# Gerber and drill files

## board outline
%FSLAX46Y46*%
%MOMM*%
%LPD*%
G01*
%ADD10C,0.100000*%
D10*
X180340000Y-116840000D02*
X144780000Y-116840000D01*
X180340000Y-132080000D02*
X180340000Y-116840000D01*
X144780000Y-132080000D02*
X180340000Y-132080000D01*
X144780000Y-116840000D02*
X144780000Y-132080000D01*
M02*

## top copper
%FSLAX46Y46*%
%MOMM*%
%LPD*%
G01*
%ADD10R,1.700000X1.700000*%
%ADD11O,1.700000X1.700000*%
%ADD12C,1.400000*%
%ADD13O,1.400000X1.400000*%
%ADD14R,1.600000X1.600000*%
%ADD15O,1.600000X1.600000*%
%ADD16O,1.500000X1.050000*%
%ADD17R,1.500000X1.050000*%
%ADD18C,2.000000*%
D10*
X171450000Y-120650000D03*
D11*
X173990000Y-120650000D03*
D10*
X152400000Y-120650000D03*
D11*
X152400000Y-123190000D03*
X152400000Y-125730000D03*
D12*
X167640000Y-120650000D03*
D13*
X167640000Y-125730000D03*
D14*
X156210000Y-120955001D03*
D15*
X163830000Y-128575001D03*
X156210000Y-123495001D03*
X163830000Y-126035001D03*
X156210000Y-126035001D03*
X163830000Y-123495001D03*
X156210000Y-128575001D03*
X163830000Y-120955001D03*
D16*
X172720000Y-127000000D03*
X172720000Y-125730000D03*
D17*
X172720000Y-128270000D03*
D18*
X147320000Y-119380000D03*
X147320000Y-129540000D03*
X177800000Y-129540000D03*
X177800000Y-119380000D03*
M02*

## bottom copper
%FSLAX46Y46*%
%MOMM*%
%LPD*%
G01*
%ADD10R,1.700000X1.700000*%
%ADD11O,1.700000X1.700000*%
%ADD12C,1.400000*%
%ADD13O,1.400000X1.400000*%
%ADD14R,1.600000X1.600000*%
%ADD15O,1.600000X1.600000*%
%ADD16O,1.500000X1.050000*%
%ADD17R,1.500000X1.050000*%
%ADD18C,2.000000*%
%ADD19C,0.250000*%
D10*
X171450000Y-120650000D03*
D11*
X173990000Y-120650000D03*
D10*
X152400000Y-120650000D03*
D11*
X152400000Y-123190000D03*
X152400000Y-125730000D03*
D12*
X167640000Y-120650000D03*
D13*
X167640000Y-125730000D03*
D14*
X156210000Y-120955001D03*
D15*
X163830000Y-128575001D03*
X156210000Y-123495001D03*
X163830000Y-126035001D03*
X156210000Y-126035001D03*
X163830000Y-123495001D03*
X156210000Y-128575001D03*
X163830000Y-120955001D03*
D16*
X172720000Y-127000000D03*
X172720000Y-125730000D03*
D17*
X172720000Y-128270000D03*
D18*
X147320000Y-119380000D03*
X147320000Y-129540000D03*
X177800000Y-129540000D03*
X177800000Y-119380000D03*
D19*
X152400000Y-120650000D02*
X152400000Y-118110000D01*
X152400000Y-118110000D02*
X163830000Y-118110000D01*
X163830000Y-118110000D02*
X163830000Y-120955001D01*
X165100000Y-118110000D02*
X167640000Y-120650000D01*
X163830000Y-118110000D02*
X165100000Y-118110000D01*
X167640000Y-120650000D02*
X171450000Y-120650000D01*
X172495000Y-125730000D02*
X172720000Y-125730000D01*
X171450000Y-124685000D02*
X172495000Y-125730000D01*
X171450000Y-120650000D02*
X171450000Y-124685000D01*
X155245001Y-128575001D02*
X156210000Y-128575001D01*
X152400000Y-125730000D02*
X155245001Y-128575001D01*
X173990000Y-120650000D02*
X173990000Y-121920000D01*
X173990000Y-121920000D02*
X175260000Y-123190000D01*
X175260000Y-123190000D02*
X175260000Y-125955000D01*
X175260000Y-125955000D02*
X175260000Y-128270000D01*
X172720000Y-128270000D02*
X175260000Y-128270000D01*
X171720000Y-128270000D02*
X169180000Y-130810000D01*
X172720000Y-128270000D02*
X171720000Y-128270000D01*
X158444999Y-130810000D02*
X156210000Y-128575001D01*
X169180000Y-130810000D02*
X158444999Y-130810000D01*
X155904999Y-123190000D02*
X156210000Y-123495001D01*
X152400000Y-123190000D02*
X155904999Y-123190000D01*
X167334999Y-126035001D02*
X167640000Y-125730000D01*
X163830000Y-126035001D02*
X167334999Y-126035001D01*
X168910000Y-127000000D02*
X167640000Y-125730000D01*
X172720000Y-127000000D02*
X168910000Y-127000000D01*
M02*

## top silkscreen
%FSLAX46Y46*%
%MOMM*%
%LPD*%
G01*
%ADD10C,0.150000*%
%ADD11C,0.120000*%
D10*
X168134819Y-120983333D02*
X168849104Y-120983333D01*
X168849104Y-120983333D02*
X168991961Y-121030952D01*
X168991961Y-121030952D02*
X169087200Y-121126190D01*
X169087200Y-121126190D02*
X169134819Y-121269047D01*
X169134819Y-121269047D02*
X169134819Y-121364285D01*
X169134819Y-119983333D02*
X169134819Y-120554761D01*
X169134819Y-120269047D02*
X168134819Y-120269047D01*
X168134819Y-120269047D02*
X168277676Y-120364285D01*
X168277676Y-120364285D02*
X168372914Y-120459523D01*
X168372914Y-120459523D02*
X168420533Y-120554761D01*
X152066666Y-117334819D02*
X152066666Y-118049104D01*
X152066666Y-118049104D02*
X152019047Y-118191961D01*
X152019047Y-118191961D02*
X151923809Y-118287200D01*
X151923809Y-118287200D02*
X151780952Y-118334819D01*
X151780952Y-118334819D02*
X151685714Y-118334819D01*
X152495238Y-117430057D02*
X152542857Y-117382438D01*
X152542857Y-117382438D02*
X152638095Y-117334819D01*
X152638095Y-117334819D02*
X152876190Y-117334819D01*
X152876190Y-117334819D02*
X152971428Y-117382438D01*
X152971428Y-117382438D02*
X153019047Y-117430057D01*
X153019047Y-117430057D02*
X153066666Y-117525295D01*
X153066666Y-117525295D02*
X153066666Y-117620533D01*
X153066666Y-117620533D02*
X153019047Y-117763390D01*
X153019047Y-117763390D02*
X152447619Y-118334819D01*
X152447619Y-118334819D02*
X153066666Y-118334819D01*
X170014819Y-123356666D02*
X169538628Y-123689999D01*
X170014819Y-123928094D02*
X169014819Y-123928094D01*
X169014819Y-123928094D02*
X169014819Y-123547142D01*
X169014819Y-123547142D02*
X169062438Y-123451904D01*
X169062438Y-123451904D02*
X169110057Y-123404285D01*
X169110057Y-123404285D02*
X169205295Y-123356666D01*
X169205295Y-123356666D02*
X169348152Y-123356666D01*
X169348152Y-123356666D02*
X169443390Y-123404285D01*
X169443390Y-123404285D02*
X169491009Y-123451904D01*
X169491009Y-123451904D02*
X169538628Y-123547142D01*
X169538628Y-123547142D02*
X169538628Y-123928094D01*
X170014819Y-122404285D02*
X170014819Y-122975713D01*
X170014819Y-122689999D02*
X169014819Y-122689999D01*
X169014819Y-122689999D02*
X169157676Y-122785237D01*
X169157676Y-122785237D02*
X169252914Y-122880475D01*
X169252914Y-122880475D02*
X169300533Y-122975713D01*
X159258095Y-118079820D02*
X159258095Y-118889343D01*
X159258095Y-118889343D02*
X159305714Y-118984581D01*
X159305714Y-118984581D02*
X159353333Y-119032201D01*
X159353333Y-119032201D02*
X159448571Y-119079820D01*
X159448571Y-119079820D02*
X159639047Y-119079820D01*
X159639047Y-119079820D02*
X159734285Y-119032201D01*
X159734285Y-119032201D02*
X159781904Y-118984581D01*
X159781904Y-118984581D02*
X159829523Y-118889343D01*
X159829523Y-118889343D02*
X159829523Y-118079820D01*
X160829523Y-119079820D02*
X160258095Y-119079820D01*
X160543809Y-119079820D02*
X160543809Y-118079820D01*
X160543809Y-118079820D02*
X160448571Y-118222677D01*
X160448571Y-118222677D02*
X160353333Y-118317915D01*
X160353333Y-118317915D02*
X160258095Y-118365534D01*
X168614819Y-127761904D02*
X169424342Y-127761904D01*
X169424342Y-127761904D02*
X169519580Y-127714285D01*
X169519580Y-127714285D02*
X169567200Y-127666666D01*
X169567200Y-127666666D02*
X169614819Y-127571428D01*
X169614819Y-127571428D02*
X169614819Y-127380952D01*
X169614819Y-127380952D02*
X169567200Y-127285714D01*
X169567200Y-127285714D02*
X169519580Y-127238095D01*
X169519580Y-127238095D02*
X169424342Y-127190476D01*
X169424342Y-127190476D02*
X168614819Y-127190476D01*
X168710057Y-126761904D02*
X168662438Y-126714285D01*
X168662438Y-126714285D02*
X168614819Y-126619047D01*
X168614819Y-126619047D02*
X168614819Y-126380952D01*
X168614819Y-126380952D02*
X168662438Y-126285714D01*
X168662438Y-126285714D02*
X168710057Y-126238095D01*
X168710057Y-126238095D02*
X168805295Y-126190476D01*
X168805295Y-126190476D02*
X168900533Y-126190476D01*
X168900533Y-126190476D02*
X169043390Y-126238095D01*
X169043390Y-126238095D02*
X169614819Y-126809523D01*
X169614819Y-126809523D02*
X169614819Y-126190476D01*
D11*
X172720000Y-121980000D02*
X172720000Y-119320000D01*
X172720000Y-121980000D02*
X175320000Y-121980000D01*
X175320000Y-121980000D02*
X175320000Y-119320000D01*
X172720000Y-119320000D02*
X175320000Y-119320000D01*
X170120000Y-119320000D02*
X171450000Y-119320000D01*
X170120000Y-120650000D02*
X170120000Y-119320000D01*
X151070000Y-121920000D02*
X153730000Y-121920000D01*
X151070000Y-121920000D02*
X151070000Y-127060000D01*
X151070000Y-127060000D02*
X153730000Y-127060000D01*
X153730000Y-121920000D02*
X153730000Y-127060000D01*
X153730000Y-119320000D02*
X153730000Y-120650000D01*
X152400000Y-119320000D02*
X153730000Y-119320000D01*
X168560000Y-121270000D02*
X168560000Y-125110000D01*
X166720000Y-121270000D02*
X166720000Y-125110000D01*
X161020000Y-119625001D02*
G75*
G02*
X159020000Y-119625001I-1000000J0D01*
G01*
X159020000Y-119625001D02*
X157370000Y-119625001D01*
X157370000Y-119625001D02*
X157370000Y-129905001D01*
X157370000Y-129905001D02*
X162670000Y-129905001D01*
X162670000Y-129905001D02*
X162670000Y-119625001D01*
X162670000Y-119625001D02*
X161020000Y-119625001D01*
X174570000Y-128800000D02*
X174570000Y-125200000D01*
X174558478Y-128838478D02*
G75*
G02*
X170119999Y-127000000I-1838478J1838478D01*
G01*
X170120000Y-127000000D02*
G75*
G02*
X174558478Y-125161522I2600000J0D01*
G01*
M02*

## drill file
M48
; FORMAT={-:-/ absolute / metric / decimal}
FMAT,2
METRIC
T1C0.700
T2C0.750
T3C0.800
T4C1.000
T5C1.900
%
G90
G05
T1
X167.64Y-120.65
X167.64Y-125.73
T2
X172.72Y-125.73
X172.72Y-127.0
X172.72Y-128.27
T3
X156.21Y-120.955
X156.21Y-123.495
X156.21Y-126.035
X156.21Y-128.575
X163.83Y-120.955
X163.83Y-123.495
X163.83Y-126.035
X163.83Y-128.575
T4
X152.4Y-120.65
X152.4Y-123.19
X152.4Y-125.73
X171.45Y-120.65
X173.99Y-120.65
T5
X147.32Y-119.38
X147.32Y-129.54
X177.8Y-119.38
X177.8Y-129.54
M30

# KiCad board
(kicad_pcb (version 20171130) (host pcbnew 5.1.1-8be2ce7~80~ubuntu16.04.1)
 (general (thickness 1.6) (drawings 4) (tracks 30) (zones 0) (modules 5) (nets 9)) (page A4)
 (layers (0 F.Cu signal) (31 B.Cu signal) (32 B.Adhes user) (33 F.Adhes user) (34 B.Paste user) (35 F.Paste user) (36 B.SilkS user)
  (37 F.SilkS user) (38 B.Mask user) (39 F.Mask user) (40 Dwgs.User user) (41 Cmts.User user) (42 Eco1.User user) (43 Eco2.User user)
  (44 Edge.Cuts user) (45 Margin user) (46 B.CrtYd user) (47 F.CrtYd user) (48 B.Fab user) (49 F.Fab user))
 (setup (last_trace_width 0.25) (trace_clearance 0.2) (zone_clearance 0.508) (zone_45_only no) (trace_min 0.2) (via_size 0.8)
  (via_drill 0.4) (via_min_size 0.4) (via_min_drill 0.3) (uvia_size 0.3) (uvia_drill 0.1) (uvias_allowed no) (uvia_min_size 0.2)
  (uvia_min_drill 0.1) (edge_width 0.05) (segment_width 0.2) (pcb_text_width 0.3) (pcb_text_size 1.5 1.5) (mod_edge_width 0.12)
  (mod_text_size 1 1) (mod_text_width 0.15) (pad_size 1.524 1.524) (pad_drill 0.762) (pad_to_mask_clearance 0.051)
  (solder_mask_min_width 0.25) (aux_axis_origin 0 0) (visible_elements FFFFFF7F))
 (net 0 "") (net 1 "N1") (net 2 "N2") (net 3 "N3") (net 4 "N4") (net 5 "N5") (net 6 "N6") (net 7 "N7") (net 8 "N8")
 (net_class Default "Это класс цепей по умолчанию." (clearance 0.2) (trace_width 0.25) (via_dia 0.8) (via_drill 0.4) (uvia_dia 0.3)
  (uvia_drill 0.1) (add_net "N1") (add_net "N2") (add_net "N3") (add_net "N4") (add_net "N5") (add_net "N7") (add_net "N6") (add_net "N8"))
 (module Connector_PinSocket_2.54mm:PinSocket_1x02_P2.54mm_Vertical (layer F.Cu) (at 171.45 120.65 90)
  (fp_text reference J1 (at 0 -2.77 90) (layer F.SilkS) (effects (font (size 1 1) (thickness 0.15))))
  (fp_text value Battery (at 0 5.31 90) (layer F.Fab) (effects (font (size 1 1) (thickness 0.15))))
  (fp_line (start -1.33 1.27) (end 1.33 1.27) (layer F.SilkS) (width 0.12))
  (fp_line (start -1.33 1.27) (end -1.33 3.87) (layer F.SilkS) (width 0.12))
  (fp_line (start -1.33 3.87) (end 1.33 3.87) (layer F.SilkS) (width 0.12))
  (fp_line (start 1.33 1.27) (end 1.33 3.87) (layer F.SilkS) (width 0.12))
  (fp_line (start 1.33 -1.33) (end 1.33 0) (layer F.SilkS) (width 0.12))
  (fp_line (start 0 -1.33) (end 1.33 -1.33) (layer F.SilkS) (width 0.12))
  (pad 1 thru_hole rect (at 0 0 90) (size 1.7 1.7) (drill 1) (layers *.Cu *.Mask) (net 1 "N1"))
  (pad 2 thru_hole oval (at 0 2.54 90) (size 1.7 1.7) (drill 1) (layers *.Cu *.Mask) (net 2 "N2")))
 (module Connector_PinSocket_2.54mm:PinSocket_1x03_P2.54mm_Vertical (layer F.Cu) (at 152.4 120.65)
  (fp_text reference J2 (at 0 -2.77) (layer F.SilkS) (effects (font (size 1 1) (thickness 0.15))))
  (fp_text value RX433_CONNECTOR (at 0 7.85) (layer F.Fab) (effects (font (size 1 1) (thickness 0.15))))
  (fp_line (start -1.33 1.27) (end 1.33 1.27) (layer F.SilkS) (width 0.12))
  (fp_line (start -1.33 1.27) (end -1.33 6.41) (layer F.SilkS) (width 0.12))
  (fp_line (start -1.33 6.41) (end 1.33 6.41) (layer F.SilkS) (width 0.12))
  (fp_line (start 1.33 1.27) (end 1.33 6.41) (layer F.SilkS) (width 0.12))
  (fp_line (start 1.33 -1.33) (end 1.33 0) (layer F.SilkS) (width 0.12))
  (fp_line (start 0 -1.33) (end 1.33 -1.33) (layer F.SilkS) (width 0.12))
  (pad 1 thru_hole rect (at 0 0) (size 1.7 1.7) (drill 1) (layers *.Cu *.Mask) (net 1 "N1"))
  (pad 2 thru_hole oval (at 0 2.54) (size 1.7 1.7) (drill 1) (layers *.Cu *.Mask) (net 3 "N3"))
  (pad 3 thru_hole oval (at 0 5.08) (size 1.7 1.7) (drill 1) (layers *.Cu *.Mask) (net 2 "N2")))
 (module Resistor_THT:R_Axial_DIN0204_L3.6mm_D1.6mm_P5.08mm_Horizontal (layer F.Cu) (at 167.64 120.65 270)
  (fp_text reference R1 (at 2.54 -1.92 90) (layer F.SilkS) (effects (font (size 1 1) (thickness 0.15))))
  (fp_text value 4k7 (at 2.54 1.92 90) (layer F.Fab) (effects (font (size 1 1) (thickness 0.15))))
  (fp_line (start 0.62 -0.92) (end 4.46 -0.92) (layer F.SilkS) (width 0.12))
  (fp_line (start 0.62 0.92) (end 4.46 0.92) (layer F.SilkS) (width 0.12))
  (pad 1 thru_hole circle (at 0 0 270) (size 1.4 1.4) (drill 0.7) (layers *.Cu *.Mask) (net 1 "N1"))
  (pad 2 thru_hole oval (at 5.08 0 270) (size 1.4 1.4) (drill 0.7) (layers *.Cu *.Mask) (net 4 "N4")))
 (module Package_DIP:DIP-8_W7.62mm (layer F.Cu) (at 156.21 120.955001)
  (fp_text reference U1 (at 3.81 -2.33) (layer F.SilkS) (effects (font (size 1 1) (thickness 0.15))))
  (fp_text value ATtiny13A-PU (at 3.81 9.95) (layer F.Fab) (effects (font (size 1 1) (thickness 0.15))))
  (fp_arc (start 3.81 -1.33) (end 2.81 -1.33) (angle -180) (layer F.SilkS) (width 0.12))
  (fp_line (start 2.81 -1.33) (end 1.16 -1.33) (layer F.SilkS) (width 0.12))
  (fp_line (start 1.16 -1.33) (end 1.16 8.95) (layer F.SilkS) (width 0.12))
  (fp_line (start 1.16 8.95) (end 6.46 8.95) (layer F.SilkS) (width 0.12))
  (fp_line (start 6.46 8.95) (end 6.46 -1.33) (layer F.SilkS) (width 0.12))
  (fp_line (start 6.46 -1.33) (end 4.81 -1.33) (layer F.SilkS) (width 0.12))
  (pad 1 thru_hole rect (at 0 0) (size 1.6 1.6) (drill 0.8) (layers *.Cu *.Mask) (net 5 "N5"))
  (pad 5 thru_hole oval (at 7.62 7.62) (size 1.6 1.6) (drill 0.8) (layers *.Cu *.Mask) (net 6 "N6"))
  (pad 2 thru_hole oval (at 0 2.54) (size 1.6 1.6) (drill 0.8) (layers *.Cu *.Mask) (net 3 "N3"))
  (pad 6 thru_hole oval (at 7.62 5.08) (size 1.6 1.6) (drill 0.8) (layers *.Cu *.Mask) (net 4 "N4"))
  (pad 3 thru_hole oval (at 0 5.08) (size 1.6 1.6) (drill 0.8) (layers *.Cu *.Mask) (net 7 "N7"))
  (pad 7 thru_hole oval (at 7.62 2.54) (size 1.6 1.6) (drill 0.8) (layers *.Cu *.Mask) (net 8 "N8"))
  (pad 4 thru_hole oval (at 0 7.62) (size 1.6 1.6) (drill 0.8) (layers *.Cu *.Mask) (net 2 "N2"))
  (pad 8 thru_hole oval (at 7.62 0) (size 1.6 1.6) (drill 0.8) (layers *.Cu *.Mask) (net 1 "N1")))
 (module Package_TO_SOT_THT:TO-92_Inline (layer F.Cu) (at 172.72 128.27 90)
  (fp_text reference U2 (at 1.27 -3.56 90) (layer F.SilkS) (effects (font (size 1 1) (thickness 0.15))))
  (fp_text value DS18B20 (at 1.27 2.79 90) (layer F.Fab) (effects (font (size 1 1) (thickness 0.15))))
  (fp_line (start -0.53 1.85) (end 3.07 1.85) (layer F.SilkS) (width 0.12))
  (fp_arc (start 1.27 0) (end 1.27 -2.6) (angle -135) (layer F.SilkS) (width 0.12))
  (fp_arc (start 1.27 0) (end 1.27 -2.6) (angle 135) (layer F.SilkS) (width 0.12))
  (pad 2 thru_hole oval (at 1.27 0 90) (size 1.05 1.5) (drill 0.75) (layers *.Cu *.Mask) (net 4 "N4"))
  (pad 3 thru_hole oval (at 2.54 0 90) (size 1.05 1.5) (drill 0.75) (layers *.Cu *.Mask) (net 1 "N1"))
  (pad 1 thru_hole rect (at 0 0 90) (size 1.05 1.5) (drill 0.75) (layers *.Cu *.Mask) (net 2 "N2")))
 (gr_line (start 180.34 116.84) (end 144.78 116.84) (layer Edge.Cuts) (width 0.1))
 (gr_line (start 180.34 132.08) (end 180.34 116.84) (layer Edge.Cuts) (width 0.1))
 (gr_line (start 144.78 132.08) (end 180.34 132.08) (layer Edge.Cuts) (width 0.1))
 (gr_line (start 144.78 116.84) (end 144.78 132.08) (layer Edge.Cuts) (width 0.1))
 (via (at 147.32 119.38) (size 2) (drill 1.9) (layers F.Cu B.Cu) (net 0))
 (via (at 147.32 129.54) (size 2) (drill 1.9) (layers F.Cu B.Cu) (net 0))
 (via (at 177.8 129.54) (size 2) (drill 1.9) (layers F.Cu B.Cu) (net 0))
 (via (at 177.8 119.38) (size 2) (drill 1.9) (layers F.Cu B.Cu) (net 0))
 (segment (start 152.4 120.65) (end 152.4 118.11) (width 0.25) (layer B.Cu) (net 1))
 (segment (start 152.4 118.11) (end 163.83 118.11) (width 0.25) (layer B.Cu) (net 1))
 (segment (start 163.83 118.11) (end 163.83 120.955001) (width 0.25) (layer B.Cu) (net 1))
 (segment (start 165.1 118.11) (end 167.64 120.65) (width 0.25) (layer B.Cu) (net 1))
 (segment (start 163.83 118.11) (end 165.1 118.11) (width 0.25) (layer B.Cu) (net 1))
 (segment (start 167.64 120.65) (end 171.45 120.65) (width 0.25) (layer B.Cu) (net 1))
 (segment (start 172.495 125.73) (end 172.72 125.73) (width 0.25) (layer B.Cu) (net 1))
 (segment (start 171.45 124.685) (end 172.495 125.73) (width 0.25) (layer B.Cu) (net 1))
 (segment (start 171.45 120.65) (end 171.45 124.685) (width 0.25) (layer B.Cu) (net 1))
 (segment (start 155.245001 128.575001) (end 156.21 128.575001) (width 0.25) (layer B.Cu) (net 2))
 (segment (start 152.4 125.73) (end 155.245001 128.575001) (width 0.25) (layer B.Cu) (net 2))
 (segment (start 173.99 120.65) (end 173.99 121.92) (width 0.25) (layer B.Cu) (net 2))
 (segment (start 173.99 121.92) (end 175.26 123.19) (width 0.25) (layer B.Cu) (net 2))
 (segment (start 175.26 123.19) (end 175.26 125.955) (width 0.25) (layer B.Cu) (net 2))
 (segment (start 175.26 125.955) (end 175.26 128.27) (width 0.25) (layer B.Cu) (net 2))
 (segment (start 172.72 128.27) (end 175.26 128.27) (width 0.25) (layer B.Cu) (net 2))
 (segment (start 171.72 128.27) (end 169.18 130.81) (width 0.25) (layer B.Cu) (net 2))
 (segment (start 172.72 128.27) (end 171.72 128.27) (width 0.25) (layer B.Cu) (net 2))
 (segment (start 158.444999 130.81) (end 156.21 128.575001) (width 0.25) (layer B.Cu) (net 2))
 (segment (start 169.18 130.81) (end 158.444999 130.81) (width 0.25) (layer B.Cu) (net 2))
 (segment (start 155.904999 123.19) (end 156.21 123.495001) (width 0.25) (layer B.Cu) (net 3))
 (segment (start 152.4 123.19) (end 155.904999 123.19) (width 0.25) (layer B.Cu) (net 3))
 (segment (start 167.334999 126.035001) (end 167.64 125.73) (width 0.25) (layer B.Cu) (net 4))
 (segment (start 163.83 126.035001) (end 167.334999 126.035001) (width 0.25) (layer B.Cu) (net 4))
 (segment (start 168.91 127) (end 167.64 125.73) (width 0.25) (layer B.Cu) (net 4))
 (segment (start 172.72 127) (end 168.91 127) (width 0.25) (layer B.Cu) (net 4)))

